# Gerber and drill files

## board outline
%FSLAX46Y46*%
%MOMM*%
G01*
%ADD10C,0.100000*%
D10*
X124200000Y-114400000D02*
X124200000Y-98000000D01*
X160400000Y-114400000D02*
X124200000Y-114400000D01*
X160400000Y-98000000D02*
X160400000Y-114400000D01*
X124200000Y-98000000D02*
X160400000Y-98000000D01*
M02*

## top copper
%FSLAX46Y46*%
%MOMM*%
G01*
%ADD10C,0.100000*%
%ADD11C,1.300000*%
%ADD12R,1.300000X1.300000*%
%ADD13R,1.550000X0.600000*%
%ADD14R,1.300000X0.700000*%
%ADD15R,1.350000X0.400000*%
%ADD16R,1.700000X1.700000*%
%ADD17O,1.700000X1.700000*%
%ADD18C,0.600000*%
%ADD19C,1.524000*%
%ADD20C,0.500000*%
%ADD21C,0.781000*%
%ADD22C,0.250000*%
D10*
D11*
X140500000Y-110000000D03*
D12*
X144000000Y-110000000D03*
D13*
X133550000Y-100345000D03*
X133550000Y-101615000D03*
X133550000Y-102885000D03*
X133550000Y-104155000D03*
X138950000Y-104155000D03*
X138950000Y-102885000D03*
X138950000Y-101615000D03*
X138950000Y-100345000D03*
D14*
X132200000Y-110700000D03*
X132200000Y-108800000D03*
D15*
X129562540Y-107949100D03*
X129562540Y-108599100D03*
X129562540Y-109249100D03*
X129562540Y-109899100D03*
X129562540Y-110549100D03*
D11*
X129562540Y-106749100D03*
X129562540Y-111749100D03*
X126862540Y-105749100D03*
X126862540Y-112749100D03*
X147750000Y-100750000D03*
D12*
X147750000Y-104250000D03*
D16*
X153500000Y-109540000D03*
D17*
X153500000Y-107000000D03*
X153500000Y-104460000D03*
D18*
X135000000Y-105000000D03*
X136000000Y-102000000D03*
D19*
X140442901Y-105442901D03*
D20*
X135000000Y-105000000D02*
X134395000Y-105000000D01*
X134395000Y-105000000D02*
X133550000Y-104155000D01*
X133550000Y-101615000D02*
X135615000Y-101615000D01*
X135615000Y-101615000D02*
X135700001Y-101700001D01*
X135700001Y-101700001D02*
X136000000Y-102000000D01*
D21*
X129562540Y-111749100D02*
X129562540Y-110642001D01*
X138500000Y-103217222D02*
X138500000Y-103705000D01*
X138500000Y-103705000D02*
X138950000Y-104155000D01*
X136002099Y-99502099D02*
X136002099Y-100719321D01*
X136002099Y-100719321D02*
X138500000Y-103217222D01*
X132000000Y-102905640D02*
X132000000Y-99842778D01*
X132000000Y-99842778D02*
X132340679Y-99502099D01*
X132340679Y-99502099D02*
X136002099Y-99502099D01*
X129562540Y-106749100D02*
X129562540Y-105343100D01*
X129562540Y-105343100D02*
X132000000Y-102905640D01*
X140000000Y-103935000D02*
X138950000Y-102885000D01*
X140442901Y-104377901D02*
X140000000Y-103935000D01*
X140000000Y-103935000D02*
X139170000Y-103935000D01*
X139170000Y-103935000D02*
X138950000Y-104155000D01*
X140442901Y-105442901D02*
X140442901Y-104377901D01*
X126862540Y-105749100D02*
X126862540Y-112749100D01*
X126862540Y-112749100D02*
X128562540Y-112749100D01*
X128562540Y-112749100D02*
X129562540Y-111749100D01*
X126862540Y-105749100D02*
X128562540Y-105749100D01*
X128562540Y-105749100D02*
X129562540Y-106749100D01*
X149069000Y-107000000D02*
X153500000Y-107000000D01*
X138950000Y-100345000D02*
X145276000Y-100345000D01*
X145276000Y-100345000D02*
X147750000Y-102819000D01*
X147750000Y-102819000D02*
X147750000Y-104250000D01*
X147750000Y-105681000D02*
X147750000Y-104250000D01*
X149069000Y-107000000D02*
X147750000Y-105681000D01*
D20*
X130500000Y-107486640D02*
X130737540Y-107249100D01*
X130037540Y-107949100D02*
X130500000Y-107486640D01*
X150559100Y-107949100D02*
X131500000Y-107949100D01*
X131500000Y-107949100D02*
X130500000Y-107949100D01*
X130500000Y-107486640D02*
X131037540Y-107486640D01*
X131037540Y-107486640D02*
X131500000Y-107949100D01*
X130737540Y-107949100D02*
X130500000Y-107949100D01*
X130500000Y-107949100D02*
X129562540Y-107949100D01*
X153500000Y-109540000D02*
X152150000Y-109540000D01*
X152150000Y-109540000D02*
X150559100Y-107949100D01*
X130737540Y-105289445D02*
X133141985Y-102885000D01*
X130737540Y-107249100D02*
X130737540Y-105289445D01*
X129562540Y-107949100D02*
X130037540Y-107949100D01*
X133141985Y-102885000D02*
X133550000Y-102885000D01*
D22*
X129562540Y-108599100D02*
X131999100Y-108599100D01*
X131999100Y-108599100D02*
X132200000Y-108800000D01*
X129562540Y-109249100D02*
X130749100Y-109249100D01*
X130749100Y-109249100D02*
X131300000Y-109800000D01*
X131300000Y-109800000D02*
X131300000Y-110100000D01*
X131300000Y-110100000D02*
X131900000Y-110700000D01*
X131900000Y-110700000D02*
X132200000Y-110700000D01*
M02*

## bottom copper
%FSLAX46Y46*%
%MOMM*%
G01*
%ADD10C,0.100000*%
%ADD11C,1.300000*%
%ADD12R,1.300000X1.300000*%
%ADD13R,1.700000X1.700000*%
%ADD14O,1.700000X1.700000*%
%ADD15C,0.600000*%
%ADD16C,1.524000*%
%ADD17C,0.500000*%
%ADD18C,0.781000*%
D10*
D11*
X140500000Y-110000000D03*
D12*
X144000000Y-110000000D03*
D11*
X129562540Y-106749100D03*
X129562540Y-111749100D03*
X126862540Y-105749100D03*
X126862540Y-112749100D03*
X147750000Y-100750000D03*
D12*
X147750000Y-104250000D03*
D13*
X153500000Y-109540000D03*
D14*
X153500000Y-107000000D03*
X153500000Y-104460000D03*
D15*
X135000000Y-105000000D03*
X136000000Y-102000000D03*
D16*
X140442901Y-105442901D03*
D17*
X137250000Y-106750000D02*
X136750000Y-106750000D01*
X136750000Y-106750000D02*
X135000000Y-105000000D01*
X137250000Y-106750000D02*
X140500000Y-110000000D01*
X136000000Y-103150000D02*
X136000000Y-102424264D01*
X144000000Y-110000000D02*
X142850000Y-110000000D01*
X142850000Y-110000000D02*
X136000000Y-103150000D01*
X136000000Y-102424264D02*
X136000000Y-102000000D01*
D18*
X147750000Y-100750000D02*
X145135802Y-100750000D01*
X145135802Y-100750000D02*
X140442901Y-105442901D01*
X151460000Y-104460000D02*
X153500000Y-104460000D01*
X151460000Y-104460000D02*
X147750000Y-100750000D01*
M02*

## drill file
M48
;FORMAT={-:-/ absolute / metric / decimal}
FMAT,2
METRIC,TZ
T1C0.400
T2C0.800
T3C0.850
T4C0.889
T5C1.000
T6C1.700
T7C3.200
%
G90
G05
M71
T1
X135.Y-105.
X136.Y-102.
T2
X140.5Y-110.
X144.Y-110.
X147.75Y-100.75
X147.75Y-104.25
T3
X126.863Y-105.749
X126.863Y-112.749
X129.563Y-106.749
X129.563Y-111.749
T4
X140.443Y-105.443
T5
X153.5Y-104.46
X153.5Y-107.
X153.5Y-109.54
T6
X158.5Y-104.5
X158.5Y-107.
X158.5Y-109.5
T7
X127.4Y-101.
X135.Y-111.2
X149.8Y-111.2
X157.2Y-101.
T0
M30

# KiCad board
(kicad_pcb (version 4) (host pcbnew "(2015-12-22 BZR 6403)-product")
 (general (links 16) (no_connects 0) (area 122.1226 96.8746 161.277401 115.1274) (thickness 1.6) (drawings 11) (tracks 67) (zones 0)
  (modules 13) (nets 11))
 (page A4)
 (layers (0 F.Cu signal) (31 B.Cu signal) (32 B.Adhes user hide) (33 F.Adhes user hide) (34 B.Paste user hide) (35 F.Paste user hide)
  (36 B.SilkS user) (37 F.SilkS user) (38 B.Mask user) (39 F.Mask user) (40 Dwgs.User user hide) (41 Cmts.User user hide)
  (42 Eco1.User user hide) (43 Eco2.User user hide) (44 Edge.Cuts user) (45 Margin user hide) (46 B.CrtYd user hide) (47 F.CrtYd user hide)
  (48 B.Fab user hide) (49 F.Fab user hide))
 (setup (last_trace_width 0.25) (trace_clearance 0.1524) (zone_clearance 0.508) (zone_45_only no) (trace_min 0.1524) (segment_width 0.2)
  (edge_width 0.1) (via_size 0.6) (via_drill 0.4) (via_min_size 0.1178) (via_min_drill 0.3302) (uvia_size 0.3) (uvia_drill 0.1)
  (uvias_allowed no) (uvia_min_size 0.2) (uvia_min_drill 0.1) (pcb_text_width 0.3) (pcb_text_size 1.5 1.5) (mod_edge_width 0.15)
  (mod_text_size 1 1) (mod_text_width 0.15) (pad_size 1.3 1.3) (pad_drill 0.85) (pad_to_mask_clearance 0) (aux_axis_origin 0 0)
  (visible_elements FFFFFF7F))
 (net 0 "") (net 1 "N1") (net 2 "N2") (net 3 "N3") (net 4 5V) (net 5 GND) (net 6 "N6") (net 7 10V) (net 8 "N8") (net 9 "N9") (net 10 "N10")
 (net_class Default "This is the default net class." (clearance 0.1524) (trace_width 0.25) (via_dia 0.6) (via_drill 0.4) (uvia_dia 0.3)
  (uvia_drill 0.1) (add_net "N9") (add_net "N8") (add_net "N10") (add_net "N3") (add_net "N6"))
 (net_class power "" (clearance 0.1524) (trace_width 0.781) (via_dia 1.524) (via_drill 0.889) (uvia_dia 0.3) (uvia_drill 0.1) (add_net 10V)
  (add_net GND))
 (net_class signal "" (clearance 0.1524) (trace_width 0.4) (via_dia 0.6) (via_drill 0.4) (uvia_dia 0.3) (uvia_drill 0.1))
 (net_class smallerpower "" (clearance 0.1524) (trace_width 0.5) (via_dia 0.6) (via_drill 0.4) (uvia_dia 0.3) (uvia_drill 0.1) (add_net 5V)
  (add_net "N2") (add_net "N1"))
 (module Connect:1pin (layer F.Cu) (at 149.8 111.2)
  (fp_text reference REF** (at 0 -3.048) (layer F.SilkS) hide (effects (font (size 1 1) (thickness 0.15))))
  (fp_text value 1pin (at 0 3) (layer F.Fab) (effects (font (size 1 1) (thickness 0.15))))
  (pad "" np_thru_hole circle (at 0 0) (size 3.2 3.2) (drill 3.2) (layers *.Cu *.SilkS F.Mask)))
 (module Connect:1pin (layer F.Cu) (at 135 111.2)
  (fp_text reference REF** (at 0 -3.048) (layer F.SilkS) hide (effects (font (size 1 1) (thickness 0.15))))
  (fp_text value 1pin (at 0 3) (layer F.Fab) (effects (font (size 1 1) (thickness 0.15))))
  (pad "" np_thru_hole circle (at 0 0) (size 3.2 3.2) (drill 3.2) (layers *.Cu *.SilkS F.Mask)))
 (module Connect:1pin (layer F.Cu) (at 127.4 101)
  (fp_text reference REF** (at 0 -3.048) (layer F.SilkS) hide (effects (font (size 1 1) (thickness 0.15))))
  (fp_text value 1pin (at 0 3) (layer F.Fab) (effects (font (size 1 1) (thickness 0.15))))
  (pad "" np_thru_hole circle (at 0 0) (size 3.2 3.2) (drill 3.2) (layers *.Cu *.SilkS F.Mask)))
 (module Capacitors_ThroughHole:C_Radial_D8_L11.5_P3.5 (layer F.Cu) (at 144 110 180)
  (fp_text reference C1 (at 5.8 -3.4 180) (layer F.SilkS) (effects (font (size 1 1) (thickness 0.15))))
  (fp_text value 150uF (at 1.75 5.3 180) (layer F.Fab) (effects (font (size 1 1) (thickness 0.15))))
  (pad 2 thru_hole circle (at 3.5 0 180) (size 1.3 1.3) (drill 0.8) (layers *.Cu *.Mask) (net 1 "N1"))
  (pad 1 thru_hole rect (at 0 0 180) (size 1.3 1.3) (drill 0.8) (layers *.Cu *.Mask) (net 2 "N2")))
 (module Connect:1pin (layer F.Cu) (at 158.5 104.5)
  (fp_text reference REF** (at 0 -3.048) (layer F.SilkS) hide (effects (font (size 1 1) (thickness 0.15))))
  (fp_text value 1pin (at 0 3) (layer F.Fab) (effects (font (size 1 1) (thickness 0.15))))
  (pad "" np_thru_hole circle (at 0 0) (size 1.7 1.7) (drill 1.7) (layers *.Cu *.Mask)))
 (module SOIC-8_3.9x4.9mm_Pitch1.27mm (layer F.Cu) (at 136.25 102.25)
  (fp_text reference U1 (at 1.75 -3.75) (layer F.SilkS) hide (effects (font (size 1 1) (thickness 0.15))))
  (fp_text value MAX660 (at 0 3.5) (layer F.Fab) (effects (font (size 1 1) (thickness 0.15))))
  (pad 1 smd rect (at -2.7 -1.905) (size 1.55 0.6) (layers F.Cu F.Paste F.Mask) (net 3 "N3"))
  (pad 2 smd rect (at -2.7 -0.635) (size 1.55 0.6) (layers F.Cu F.Paste F.Mask) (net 2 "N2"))
  (pad 3 smd rect (at -2.7 0.635) (size 1.55 0.6) (layers F.Cu F.Paste F.Mask) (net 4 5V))
  (pad 4 smd rect (at -2.7 1.905) (size 1.55 0.6) (layers F.Cu F.Paste F.Mask) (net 1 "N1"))
  (pad 5 smd rect (at 2.7 1.905) (size 1.55 0.6) (layers F.Cu F.Paste F.Mask) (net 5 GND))
  (pad 6 smd rect (at 2.7 0.635) (size 1.55 0.6) (layers F.Cu F.Paste F.Mask) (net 5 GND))
  (pad 7 smd rect (at 2.7 -0.635) (size 1.55 0.6) (layers F.Cu F.Paste F.Mask) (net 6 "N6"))
  (pad 8 smd rect (at 2.7 -1.905) (size 1.55 0.6) (layers F.Cu F.Paste F.Mask) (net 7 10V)))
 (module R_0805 (layer F.Cu) (at 132.2 109.75 90)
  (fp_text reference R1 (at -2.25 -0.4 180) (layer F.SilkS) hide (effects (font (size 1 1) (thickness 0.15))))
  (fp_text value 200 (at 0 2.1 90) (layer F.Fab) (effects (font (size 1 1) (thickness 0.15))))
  (pad 1 smd rect (at -0.95 0 90) (size 0.7 1.3) (layers F.Cu F.Paste F.Mask) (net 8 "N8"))
  (pad 2 smd rect (at 0.95 0 90) (size 0.7 1.3) (layers F.Cu F.Paste F.Mask) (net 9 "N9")))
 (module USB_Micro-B (layer F.Cu) (at 128 109.25 270)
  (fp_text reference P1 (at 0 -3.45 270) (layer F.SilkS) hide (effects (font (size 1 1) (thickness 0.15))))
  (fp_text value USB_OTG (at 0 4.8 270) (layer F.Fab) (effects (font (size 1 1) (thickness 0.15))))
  (pad 1 smd rect (at -1.3009 -1.56254) (size 1.35 0.4) (layers F.Cu F.Paste F.Mask) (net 4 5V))
  (pad 2 smd rect (at -0.6509 -1.56254) (size 1.35 0.4) (layers F.Cu F.Paste F.Mask) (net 9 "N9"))
  (pad 3 smd rect (at -0.0009 -1.56254) (size 1.35 0.4) (layers F.Cu F.Paste F.Mask) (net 8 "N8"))
  (pad 4 smd rect (at 0.6491 -1.56254) (size 1.35 0.4) (layers F.Cu F.Paste F.Mask) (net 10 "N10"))
  (pad 5 smd rect (at 1.2991 -1.56254) (size 1.35 0.4) (layers F.Cu F.Paste F.Mask) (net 5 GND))
  (pad 6 thru_hole circle (at -2.5009 -1.56254) (size 1.3 1.3) (drill 0.85) (layers *.Cu *.Mask) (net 5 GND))
  (pad 6 thru_hole circle (at 2.4991 -1.56254) (size 1.3 1.3) (drill 0.85) (layers *.Cu *.Mask) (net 5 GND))
  (pad 6 thru_hole circle (at -3.5009 1.13746) (size 1.3 1.3) (drill 0.85) (layers *.Cu *.Mask) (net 5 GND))
  (pad 6 thru_hole circle (at 3.4991 1.13746) (size 1.3 1.3) (drill 0.85) (layers *.Cu *.Mask) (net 5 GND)))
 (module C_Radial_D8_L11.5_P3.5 (layer F.Cu) (at 147.75 104.25 90)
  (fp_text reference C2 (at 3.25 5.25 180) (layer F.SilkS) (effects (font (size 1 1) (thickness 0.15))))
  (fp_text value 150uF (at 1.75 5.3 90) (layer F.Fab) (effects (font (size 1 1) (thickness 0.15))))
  (pad 2 thru_hole circle (at 3.5 0 90) (size 1.3 1.3) (drill 0.8) (layers *.Cu *.Mask) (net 5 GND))
  (pad 1 thru_hole rect (at 0 0 90) (size 1.3 1.3) (drill 0.8) (layers *.Cu *.Mask) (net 7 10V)))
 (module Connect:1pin (layer F.Cu) (at 158.5 107)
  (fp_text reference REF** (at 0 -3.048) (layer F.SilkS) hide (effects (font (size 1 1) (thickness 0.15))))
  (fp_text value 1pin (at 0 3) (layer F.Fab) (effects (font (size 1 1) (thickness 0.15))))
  (pad "" np_thru_hole circle (at 0 0) (size 1.7 1.7) (drill 1.7) (layers *.Cu *.Mask F.SilkS)))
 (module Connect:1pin (layer F.Cu) (at 158.5 109.5)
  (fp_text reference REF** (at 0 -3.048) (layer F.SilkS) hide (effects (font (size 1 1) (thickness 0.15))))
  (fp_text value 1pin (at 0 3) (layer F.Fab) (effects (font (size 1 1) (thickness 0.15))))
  (pad "" np_thru_hole circle (at 0 0) (size 1.7 1.7) (drill 1.7) (layers *.Cu *.Mask F.SilkS)))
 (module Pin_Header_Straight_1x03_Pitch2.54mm (layer F.Cu) (at 153.5 109.54 180)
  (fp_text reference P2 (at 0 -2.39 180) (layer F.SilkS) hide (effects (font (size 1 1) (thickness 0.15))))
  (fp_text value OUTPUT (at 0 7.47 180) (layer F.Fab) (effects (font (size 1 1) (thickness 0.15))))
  (pad 1 thru_hole rect (at 0 0 180) (size 1.7 1.7) (drill 1) (layers *.Cu *.Mask) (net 4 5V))
  (pad 2 thru_hole oval (at 0 2.54 180) (size 1.7 1.7) (drill 1) (layers *.Cu *.Mask) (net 7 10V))
  (pad 3 thru_hole oval (at 0 5.08 180) (size 1.7 1.7) (drill 1) (layers *.Cu *.Mask) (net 5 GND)))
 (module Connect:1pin (layer F.Cu) (at 157.2 101)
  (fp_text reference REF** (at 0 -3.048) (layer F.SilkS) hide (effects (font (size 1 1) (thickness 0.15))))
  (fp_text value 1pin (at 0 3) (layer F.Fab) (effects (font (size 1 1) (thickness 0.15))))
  (pad "" np_thru_hole circle (at 0 0) (size 3.2 3.2) (drill 3.2) (layers *.Cu *.SilkS F.Mask)))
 (gr_line (start 124.2 114.4) (end 124.2 98) (layer Edge.Cuts) (width 0.1))
 (gr_line (start 160.4 114.4) (end 124.2 114.4) (layer Edge.Cuts) (width 0.1))
 (gr_line (start 160.4 98) (end 160.4 114.4) (layer Edge.Cuts) (width 0.1))
 (gr_line (start 124.2 98) (end 160.4 98) (layer Edge.Cuts) (width 0.1))
 (segment (start 124.2 98.2) (end 124.2 98) (width 0.25) (layer Dwgs.User) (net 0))
 (segment (start 137.25 106.75) (end 136.75 106.75) (width 0.5) (layer B.Cu) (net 1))
 (segment (start 136.75 106.75) (end 135 105) (width 0.5) (layer B.Cu) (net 1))
 (segment (start 137.25 106.75) (end 140.5 110) (width 0.5) (layer B.Cu) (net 1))
 (segment (start 135 105) (end 134.395 105) (width 0.5) (layer F.Cu) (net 1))
 (segment (start 134.395 105) (end 133.55 104.155) (width 0.5) (layer F.Cu) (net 1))
 (via (at 135 105) (size 0.6) (drill 0.4) (layers F.Cu B.Cu) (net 1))
 (segment (start 136 103.15) (end 136 102.424264) (width 0.5) (layer B.Cu) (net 2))
 (segment (start 144 110) (end 142.85 110) (width 0.5) (layer B.Cu) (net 2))
 (segment (start 142.85 110) (end 136 103.15) (width 0.5) (layer B.Cu) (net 2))
 (segment (start 136 102.424264) (end 136 102) (width 0.5) (layer B.Cu) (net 2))
 (segment (start 133.55 101.615) (end 135.615 101.615) (width 0.5) (layer F.Cu) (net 2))
 (segment (start 135.615 101.615) (end 135.700001 101.700001) (width 0.5) (layer F.Cu) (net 2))
 (segment (start 135.700001 101.700001) (end 136 102) (width 0.5) (layer F.Cu) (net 2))
 (via (at 136 102) (size 0.6) (drill 0.4) (layers F.Cu B.Cu) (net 2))
 (segment (start 147.75 100.75) (end 145.135802 100.75) (width 0.781) (layer B.Cu) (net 5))
 (segment (start 145.135802 100.75) (end 140.442901 105.442901) (width 0.781) (layer B.Cu) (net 5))
 (segment (start 151.46 104.46) (end 153.5 104.46) (width 0.781) (layer B.Cu) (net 5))
 (segment (start 129.56254 111.7491) (end 129.56254 110.642001) (width 0.781) (layer F.Cu) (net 5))
 (segment (start 138.5 103.217222) (end 138.5 103.705) (width 0.781) (layer F.Cu) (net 5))
 (segment (start 138.5 103.705) (end 138.95 104.155) (width 0.781) (layer F.Cu) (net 5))
 (segment (start 136.002099 99.502099) (end 136.002099 100.719321) (width 0.781) (layer F.Cu) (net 5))
 (segment (start 136.002099 100.719321) (end 138.5 103.217222) (width 0.781) (layer F.Cu) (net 5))
 (segment (start 132 102.90564) (end 132 99.842778) (width 0.781) (layer F.Cu) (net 5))
 (segment (start 132 99.842778) (end 132.340679 99.502099) (width 0.781) (layer F.Cu) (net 5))
 (segment (start 132.340679 99.502099) (end 136.002099 99.502099) (width 0.781) (layer F.Cu) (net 5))
 (segment (start 129.56254 106.7491) (end 129.56254 105.3431) (width 0.781) (layer F.Cu) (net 5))
 (segment (start 129.56254 105.3431) (end 132 102.90564) (width 0.781) (layer F.Cu) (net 5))
 (segment (start 140 103.935) (end 138.95 102.885) (width 0.781) (layer F.Cu) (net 5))
 (segment (start 140.442901 104.377901) (end 140 103.935) (width 0.781) (layer F.Cu) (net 5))
 (segment (start 140 103.935) (end 139.17 103.935) (width 0.781) (layer F.Cu) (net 5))
 (segment (start 139.17 103.935) (end 138.95 104.155) (width 0.781) (layer F.Cu) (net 5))
 (segment (start 140.442901 105.442901) (end 140.442901 104.377901) (width 0.781) (layer F.Cu) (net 5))
 (via (at 140.442901 105.442901) (size 1.524) (drill 0.889) (layers F.Cu B.Cu) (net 5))
 (segment (start 151.46 104.46) (end 147.75 100.75) (width 0.781) (layer B.Cu) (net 5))
 (segment (start 126.86254 105.7491) (end 126.86254 112.7491) (width 0.781) (layer F.Cu) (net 5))
 (segment (start 126.86254 112.7491) (end 128.56254 112.7491) (width 0.781) (layer F.Cu) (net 5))
 (segment (start 128.56254 112.7491) (end 129.56254 111.7491) (width 0.781) (layer F.Cu) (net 5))
 (segment (start 126.86254 105.7491) (end 128.56254 105.7491) (width 0.781) (layer F.Cu) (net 5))
 (segment (start 128.56254 105.7491) (end 129.56254 106.7491) (width 0.781) (layer F.Cu) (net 5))
 (segment (start 149.069 107) (end 153.5 107) (width 0.781) (layer F.Cu) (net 7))
 (segment (start 138.95 100.345) (end 145.276 100.345) (width 0.781) (layer F.Cu) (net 7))
 (segment (start 145.276 100.345) (end 147.75 102.819) (width 0.781) (layer F.Cu) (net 7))
 (segment (start 147.75 102.819) (end 147.75 104.25) (width 0.781) (layer F.Cu) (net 7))
 (segment (start 147.75 105.681) (end 147.75 104.25) (width 0.781) (layer F.Cu) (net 7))
 (segment (start 149.069 107) (end 147.75 105.681) (width 0.781) (layer F.Cu) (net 7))
 (segment (start 130.5 107.48664) (end 130.73754 107.2491) (width 0.5) (layer F.Cu) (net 4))
 (segment (start 130.03754 107.9491) (end 130.5 107.48664) (width 0.5) (layer F.Cu) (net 4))
 (segment (start 150.5591 107.9491) (end 131.5 107.9491) (width 0.5) (layer F.Cu) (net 4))
 (segment (start 131.5 107.9491) (end 130.5 107.9491) (width 0.5) (layer F.Cu) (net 4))
 (segment (start 130.5 107.48664) (end 131.03754 107.48664) (width 0.5) (layer F.Cu) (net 4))
 (segment (start 131.03754 107.48664) (end 131.5 107.9491) (width 0.5) (layer F.Cu) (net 4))
 (segment (start 130.73754 107.9491) (end 130.5 107.9491) (width 0.5) (layer F.Cu) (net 4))
 (segment (start 130.5 107.9491) (end 129.56254 107.9491) (width 0.5) (layer F.Cu) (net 4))
 (segment (start 153.5 109.54) (end 152.15 109.54) (width 0.5) (layer F.Cu) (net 4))
 (segment (start 152.15 109.54) (end 150.5591 107.9491) (width 0.5) (layer F.Cu) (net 4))
 (segment (start 130.73754 105.289445) (end 133.141985 102.885) (width 0.5) (layer F.Cu) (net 4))
 (segment (start 130.73754 107.2491) (end 130.73754 105.289445) (width 0.5) (layer F.Cu) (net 4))
 (segment (start 129.56254 107.9491) (end 130.03754 107.9491) (width 0.5) (layer F.Cu) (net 4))
 (segment (start 133.141985 102.885) (end 133.55 102.885) (width 0.5) (layer F.Cu) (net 4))
 (segment (start 129.56254 108.5991) (end 131.9991 108.5991) (width 0.25) (layer F.Cu) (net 9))
 (segment (start 131.9991 108.5991) (end 132.2 108.8) (width 0.25) (layer F.Cu) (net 9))
 (segment (start 129.56254 109.2491) (end 130.7491 109.2491) (width 0.25) (layer F.Cu) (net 8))
 (segment (start 130.7491 109.2491) (end 131.3 109.8) (width 0.25) (layer F.Cu) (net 8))
 (segment (start 131.3 109.8) (end 131.3 110.1) (width 0.25) (layer F.Cu) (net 8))
 (segment (start 131.3 110.1) (end 131.9 110.7) (width 0.25) (layer F.Cu) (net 8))
 (segment (start 131.9 110.7) (end 132.2 110.7) (width 0.25) (layer F.Cu) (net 8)))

